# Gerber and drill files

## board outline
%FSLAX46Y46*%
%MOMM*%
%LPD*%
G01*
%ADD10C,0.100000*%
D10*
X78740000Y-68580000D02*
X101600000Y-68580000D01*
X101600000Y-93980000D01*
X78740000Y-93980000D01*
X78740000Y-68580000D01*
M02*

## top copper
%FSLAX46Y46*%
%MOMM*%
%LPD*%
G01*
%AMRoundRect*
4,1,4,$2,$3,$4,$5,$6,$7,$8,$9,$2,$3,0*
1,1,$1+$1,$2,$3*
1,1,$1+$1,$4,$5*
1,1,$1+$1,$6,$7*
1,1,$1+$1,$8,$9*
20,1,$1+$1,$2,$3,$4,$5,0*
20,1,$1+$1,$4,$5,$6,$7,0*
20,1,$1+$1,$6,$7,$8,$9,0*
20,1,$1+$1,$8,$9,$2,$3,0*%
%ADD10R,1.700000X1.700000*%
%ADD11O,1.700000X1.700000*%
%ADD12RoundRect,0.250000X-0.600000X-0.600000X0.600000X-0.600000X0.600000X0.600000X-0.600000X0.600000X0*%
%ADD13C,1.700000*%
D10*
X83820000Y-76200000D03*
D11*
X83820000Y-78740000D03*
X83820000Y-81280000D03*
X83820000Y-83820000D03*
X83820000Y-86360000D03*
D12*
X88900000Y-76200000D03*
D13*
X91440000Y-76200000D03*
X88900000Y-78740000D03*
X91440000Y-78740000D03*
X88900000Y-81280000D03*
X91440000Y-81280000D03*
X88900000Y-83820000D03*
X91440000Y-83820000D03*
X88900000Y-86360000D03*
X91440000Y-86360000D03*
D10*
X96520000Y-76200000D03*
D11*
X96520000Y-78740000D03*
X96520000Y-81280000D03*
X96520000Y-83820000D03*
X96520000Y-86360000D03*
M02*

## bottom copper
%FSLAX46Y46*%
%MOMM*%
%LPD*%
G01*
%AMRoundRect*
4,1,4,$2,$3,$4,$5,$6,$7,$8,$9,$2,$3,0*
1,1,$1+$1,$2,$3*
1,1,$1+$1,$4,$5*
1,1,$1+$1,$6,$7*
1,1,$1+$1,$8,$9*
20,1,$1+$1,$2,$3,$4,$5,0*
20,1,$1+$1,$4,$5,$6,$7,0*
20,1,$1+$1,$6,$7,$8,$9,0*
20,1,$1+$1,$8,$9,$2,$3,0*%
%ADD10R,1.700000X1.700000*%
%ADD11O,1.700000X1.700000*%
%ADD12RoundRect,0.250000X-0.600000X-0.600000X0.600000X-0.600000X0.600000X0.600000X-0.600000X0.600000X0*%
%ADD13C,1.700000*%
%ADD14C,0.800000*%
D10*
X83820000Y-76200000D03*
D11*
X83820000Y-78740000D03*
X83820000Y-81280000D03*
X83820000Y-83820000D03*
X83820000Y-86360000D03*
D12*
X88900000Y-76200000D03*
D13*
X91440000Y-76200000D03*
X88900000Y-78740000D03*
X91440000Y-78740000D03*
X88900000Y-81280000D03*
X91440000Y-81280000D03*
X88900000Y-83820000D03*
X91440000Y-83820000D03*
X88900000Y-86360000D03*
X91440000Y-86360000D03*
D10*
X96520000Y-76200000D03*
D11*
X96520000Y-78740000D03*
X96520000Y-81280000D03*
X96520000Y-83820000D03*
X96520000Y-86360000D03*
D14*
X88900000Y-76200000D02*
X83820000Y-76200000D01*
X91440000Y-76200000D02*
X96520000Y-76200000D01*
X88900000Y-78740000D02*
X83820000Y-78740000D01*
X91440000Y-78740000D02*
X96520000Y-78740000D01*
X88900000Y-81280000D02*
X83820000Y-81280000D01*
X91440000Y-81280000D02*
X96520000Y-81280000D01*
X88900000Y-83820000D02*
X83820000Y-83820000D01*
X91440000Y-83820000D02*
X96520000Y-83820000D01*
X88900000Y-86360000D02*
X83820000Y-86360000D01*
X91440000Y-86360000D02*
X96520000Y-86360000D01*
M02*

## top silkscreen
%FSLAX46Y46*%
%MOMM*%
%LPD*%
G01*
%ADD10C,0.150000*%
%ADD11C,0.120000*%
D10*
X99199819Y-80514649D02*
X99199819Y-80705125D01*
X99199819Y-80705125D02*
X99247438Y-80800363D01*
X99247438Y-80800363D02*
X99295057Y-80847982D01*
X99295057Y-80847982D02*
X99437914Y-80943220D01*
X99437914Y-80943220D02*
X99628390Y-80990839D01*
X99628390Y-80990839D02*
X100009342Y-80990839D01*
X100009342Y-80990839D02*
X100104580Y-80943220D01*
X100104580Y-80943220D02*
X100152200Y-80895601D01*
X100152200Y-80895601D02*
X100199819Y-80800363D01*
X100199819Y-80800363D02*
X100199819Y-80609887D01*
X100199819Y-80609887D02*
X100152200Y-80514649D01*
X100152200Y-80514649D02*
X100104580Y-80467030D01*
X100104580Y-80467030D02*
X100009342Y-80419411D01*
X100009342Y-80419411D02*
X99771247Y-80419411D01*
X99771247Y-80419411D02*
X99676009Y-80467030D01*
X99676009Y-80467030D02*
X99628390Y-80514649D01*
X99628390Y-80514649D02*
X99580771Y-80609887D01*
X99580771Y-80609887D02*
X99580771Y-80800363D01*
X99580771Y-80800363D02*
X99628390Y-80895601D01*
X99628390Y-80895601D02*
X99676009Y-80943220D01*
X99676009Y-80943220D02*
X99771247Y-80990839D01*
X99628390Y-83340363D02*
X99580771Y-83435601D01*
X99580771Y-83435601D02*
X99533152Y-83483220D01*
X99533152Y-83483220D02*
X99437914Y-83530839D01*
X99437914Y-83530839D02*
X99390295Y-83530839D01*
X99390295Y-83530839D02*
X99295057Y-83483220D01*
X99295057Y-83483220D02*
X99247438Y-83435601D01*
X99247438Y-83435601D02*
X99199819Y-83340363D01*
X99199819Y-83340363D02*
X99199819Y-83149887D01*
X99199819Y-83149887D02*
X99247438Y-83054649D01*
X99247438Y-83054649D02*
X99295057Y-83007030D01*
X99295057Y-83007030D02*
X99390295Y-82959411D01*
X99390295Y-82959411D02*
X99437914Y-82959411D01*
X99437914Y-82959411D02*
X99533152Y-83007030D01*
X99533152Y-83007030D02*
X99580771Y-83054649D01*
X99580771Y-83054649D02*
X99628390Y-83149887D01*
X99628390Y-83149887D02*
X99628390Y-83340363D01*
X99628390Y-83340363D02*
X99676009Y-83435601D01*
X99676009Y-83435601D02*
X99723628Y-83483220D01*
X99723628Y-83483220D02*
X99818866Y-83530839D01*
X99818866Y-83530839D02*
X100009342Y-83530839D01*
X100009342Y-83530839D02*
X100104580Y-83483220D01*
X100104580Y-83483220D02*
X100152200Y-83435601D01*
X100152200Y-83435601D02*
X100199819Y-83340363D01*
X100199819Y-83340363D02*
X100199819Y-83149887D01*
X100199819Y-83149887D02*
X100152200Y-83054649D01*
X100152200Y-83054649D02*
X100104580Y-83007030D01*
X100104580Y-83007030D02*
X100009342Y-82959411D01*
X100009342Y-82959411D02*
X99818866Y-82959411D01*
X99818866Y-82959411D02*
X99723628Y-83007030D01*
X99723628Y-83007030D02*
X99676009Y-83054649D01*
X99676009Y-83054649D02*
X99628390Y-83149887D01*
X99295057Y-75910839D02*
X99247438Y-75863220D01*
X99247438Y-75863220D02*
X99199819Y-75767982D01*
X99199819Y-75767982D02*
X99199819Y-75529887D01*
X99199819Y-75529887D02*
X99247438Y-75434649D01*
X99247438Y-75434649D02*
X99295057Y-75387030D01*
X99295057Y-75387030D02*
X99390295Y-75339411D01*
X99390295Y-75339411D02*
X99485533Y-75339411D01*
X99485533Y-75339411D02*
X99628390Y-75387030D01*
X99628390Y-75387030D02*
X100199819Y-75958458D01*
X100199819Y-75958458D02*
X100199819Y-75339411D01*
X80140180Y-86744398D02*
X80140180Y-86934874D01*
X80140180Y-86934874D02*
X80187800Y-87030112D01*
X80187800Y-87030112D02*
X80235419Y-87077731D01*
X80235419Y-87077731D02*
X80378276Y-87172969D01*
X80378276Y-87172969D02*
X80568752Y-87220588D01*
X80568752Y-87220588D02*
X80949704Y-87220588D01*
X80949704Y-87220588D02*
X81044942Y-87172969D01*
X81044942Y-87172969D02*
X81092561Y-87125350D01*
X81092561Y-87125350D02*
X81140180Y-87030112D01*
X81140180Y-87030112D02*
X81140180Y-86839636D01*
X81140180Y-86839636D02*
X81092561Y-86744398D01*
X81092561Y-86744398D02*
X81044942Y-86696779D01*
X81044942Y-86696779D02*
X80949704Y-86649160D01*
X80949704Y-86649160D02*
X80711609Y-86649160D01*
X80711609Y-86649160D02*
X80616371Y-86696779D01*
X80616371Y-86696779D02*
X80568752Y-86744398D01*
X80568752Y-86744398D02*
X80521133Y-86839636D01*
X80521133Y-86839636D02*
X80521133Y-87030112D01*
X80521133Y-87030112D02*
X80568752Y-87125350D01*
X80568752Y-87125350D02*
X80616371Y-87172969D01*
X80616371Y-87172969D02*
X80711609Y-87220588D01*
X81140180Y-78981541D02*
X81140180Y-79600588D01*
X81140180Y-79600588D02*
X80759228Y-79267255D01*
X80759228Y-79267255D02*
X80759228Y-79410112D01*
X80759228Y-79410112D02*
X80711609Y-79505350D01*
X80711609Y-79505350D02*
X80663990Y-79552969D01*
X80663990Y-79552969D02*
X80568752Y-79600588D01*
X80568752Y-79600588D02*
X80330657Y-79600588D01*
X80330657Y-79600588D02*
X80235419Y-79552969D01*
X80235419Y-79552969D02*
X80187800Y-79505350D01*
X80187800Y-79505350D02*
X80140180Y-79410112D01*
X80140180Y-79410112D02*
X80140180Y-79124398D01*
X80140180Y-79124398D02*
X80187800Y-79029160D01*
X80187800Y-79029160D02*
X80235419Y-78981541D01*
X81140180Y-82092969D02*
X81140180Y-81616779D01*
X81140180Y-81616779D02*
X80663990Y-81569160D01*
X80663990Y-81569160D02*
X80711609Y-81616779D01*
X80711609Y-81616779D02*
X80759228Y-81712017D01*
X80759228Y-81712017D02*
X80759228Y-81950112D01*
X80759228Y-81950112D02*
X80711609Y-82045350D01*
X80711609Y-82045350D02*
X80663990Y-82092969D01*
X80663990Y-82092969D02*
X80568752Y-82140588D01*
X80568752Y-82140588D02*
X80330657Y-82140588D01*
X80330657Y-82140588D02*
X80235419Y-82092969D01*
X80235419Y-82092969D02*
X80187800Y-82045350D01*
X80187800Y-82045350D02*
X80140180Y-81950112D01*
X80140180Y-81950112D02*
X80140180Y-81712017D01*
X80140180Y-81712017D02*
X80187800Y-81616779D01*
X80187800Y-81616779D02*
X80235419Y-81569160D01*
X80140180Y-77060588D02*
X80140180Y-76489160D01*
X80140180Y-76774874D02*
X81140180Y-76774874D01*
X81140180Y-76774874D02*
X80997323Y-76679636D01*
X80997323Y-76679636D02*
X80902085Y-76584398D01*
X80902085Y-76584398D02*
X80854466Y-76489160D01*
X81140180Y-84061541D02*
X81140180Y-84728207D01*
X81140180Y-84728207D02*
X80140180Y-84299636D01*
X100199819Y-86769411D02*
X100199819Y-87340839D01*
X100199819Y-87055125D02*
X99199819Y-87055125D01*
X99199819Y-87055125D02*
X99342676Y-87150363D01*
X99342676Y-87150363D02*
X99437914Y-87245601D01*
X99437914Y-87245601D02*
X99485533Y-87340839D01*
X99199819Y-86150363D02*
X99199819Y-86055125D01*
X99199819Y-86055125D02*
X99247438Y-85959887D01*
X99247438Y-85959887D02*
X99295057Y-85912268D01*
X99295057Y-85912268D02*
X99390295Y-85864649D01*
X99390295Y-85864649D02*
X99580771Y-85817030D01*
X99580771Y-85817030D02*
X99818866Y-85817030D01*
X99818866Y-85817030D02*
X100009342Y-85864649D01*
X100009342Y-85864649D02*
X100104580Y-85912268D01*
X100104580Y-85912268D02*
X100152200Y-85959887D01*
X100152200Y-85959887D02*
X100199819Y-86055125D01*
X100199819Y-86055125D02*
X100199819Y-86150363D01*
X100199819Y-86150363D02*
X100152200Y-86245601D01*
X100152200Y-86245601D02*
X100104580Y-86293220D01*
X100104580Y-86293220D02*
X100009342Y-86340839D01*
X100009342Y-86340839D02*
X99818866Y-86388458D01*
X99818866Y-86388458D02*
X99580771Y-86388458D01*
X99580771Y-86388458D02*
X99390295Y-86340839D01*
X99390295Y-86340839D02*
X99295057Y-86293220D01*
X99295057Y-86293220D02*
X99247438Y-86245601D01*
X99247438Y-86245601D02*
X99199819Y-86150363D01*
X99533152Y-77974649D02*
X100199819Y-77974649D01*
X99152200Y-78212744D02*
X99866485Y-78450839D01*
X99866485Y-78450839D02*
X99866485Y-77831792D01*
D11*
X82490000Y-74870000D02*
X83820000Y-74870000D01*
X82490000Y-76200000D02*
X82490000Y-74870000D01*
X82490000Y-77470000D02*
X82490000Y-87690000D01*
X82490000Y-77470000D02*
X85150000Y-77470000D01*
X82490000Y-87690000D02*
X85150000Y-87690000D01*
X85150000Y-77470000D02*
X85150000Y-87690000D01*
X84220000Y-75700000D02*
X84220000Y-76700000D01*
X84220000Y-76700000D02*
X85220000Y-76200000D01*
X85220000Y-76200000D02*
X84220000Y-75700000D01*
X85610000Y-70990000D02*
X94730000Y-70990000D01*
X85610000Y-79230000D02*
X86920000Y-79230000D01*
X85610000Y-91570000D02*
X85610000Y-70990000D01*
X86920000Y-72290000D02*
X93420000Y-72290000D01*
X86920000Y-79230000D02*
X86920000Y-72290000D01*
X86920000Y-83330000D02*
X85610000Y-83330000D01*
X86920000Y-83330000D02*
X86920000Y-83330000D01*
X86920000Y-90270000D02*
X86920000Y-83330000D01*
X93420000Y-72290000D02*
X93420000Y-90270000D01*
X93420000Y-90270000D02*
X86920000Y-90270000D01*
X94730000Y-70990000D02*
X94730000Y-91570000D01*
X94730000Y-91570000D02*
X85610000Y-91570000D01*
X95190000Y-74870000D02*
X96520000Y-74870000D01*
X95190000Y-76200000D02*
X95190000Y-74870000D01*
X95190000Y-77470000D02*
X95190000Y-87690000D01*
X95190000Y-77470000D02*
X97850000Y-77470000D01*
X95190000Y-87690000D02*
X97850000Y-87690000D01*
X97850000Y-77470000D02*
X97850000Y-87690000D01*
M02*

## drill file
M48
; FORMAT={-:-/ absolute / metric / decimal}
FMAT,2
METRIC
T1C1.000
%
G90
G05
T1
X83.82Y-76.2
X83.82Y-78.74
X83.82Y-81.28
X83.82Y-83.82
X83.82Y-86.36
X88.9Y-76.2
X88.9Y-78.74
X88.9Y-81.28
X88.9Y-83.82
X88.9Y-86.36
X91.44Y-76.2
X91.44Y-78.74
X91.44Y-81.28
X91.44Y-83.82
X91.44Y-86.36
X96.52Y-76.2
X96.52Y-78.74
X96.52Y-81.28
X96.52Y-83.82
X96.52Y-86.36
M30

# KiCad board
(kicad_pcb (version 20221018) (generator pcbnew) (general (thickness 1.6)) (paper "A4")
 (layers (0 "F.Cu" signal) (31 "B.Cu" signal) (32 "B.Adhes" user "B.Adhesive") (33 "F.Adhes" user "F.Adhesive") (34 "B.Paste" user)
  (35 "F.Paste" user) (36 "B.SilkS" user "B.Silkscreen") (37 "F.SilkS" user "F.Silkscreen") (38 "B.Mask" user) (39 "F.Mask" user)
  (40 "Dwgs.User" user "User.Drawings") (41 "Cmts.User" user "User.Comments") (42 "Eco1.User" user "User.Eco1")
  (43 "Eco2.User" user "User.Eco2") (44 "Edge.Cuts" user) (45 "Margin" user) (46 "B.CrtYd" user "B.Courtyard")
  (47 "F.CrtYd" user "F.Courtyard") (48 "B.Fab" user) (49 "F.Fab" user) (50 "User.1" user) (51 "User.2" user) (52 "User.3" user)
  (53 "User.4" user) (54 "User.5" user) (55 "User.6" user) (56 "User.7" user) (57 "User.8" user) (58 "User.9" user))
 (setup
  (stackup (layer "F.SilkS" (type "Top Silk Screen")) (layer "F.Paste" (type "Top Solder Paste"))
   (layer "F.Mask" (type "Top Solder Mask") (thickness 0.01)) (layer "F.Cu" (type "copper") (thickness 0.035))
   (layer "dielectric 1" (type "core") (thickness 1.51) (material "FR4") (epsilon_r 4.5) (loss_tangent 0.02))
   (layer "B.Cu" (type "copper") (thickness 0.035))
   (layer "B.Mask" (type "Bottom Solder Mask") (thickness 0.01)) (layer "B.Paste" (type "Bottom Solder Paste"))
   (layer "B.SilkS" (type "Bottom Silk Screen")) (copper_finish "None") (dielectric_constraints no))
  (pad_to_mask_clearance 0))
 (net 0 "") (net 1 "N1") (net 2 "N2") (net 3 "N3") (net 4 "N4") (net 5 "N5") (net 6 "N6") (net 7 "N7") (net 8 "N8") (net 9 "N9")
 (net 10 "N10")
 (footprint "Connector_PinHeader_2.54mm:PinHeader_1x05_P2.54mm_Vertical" (layer "F.Cu") (at 83.82 76.2)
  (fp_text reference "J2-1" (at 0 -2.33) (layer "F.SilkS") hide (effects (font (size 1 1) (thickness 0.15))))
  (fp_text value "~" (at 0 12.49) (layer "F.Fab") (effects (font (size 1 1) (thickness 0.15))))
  (fp_line (start -1.33 -1.33) (end 0 -1.33) (stroke (width 0.12) (type solid)) (layer "F.SilkS"))
  (fp_line (start -1.33 0) (end -1.33 -1.33) (stroke (width 0.12) (type solid)) (layer "F.SilkS"))
  (fp_line (start -1.33 1.27) (end -1.33 11.49) (stroke (width 0.12) (type solid)) (layer "F.SilkS"))
  (fp_line (start -1.33 1.27) (end 1.33 1.27) (stroke (width 0.12) (type solid)) (layer "F.SilkS"))
  (fp_line (start -1.33 11.49) (end 1.33 11.49) (stroke (width 0.12) (type solid)) (layer "F.SilkS"))
  (fp_line (start 1.33 1.27) (end 1.33 11.49) (stroke (width 0.12) (type solid)) (layer "F.SilkS"))
  (pad "1" thru_hole rect (at 0 0) (size 1.7 1.7) (drill 1) (layers "*.Cu" "*.Mask") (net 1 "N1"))
  (pad "2" thru_hole oval (at 0 2.54) (size 1.7 1.7) (drill 1) (layers "*.Cu" "*.Mask") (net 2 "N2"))
  (pad "3" thru_hole oval (at 0 5.08) (size 1.7 1.7) (drill 1) (layers "*.Cu" "*.Mask") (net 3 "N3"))
  (pad "4" thru_hole oval (at 0 7.62) (size 1.7 1.7) (drill 1) (layers "*.Cu" "*.Mask") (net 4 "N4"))
  (pad "5" thru_hole oval (at 0 10.16) (size 1.7 1.7) (drill 1) (layers "*.Cu" "*.Mask") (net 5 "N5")))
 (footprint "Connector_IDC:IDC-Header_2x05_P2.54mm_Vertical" (layer "F.Cu") (at 88.9 76.2)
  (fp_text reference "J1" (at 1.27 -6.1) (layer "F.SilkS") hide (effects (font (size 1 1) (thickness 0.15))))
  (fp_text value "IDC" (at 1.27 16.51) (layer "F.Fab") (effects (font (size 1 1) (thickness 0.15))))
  (fp_line (start -4.68 -0.5) (end -4.68 0.5) (stroke (width 0.12) (type solid)) (layer "F.SilkS"))
  (fp_line (start -4.68 0.5) (end -3.68 0) (stroke (width 0.12) (type solid)) (layer "F.SilkS"))
  (fp_line (start -3.68 0) (end -4.68 -0.5) (stroke (width 0.12) (type solid)) (layer "F.SilkS"))
  (fp_line (start -3.29 -5.21) (end 5.83 -5.21) (stroke (width 0.12) (type solid)) (layer "F.SilkS"))
  (fp_line (start -3.29 3.03) (end -1.98 3.03) (stroke (width 0.12) (type solid)) (layer "F.SilkS"))
  (fp_line (start -3.29 15.37) (end -3.29 -5.21) (stroke (width 0.12) (type solid)) (layer "F.SilkS"))
  (fp_line (start -1.98 -3.91) (end 4.52 -3.91) (stroke (width 0.12) (type solid)) (layer "F.SilkS"))
  (fp_line (start -1.98 3.03) (end -1.98 -3.91) (stroke (width 0.12) (type solid)) (layer "F.SilkS"))
  (fp_line (start -1.98 7.13) (end -3.29 7.13) (stroke (width 0.12) (type solid)) (layer "F.SilkS"))
  (fp_line (start -1.98 7.13) (end -1.98 7.13) (stroke (width 0.12) (type solid)) (layer "F.SilkS"))
  (fp_line (start -1.98 14.07) (end -1.98 7.13) (stroke (width 0.12) (type solid)) (layer "F.SilkS"))
  (fp_line (start 4.52 -3.91) (end 4.52 14.07) (stroke (width 0.12) (type solid)) (layer "F.SilkS"))
  (fp_line (start 4.52 14.07) (end -1.98 14.07) (stroke (width 0.12) (type solid)) (layer "F.SilkS"))
  (fp_line (start 5.83 -5.21) (end 5.83 15.37) (stroke (width 0.12) (type solid)) (layer "F.SilkS"))
  (fp_line (start 5.83 15.37) (end -3.29 15.37) (stroke (width 0.12) (type solid)) (layer "F.SilkS"))
  (pad "1" thru_hole roundrect (at 0 0) (size 1.7 1.7) (drill 1) (layers "*.Cu" "*.Mask") (roundrect_rratio 0.147059) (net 1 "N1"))
  (pad "2" thru_hole circle (at 2.54 0) (size 1.7 1.7) (drill 1) (layers "*.Cu" "*.Mask") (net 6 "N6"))
  (pad "3" thru_hole circle (at 0 2.54) (size 1.7 1.7) (drill 1) (layers "*.Cu" "*.Mask") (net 2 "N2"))
  (pad "4" thru_hole circle (at 2.54 2.54) (size 1.7 1.7) (drill 1) (layers "*.Cu" "*.Mask") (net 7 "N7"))
  (pad "5" thru_hole circle (at 0 5.08) (size 1.7 1.7) (drill 1) (layers "*.Cu" "*.Mask") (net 3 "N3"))
  (pad "6" thru_hole circle (at 2.54 5.08) (size 1.7 1.7) (drill 1) (layers "*.Cu" "*.Mask") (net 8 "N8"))
  (pad "7" thru_hole circle (at 0 7.62) (size 1.7 1.7) (drill 1) (layers "*.Cu" "*.Mask") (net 4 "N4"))
  (pad "8" thru_hole circle (at 2.54 7.62) (size 1.7 1.7) (drill 1) (layers "*.Cu" "*.Mask") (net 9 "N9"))
  (pad "9" thru_hole circle (at 0 10.16) (size 1.7 1.7) (drill 1) (layers "*.Cu" "*.Mask") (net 5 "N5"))
  (pad "10" thru_hole circle (at 2.54 10.16) (size 1.7 1.7) (drill 1) (layers "*.Cu" "*.Mask") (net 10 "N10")))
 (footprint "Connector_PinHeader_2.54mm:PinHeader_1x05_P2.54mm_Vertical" (layer "F.Cu") (at 96.52 76.2)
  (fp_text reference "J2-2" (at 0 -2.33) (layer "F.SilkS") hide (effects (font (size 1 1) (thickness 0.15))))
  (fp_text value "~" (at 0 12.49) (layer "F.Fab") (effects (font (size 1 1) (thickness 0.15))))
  (fp_line (start -1.33 -1.33) (end 0 -1.33) (stroke (width 0.12) (type solid)) (layer "F.SilkS"))
  (fp_line (start -1.33 0) (end -1.33 -1.33) (stroke (width 0.12) (type solid)) (layer "F.SilkS"))
  (fp_line (start -1.33 1.27) (end -1.33 11.49) (stroke (width 0.12) (type solid)) (layer "F.SilkS"))
  (fp_line (start -1.33 1.27) (end 1.33 1.27) (stroke (width 0.12) (type solid)) (layer "F.SilkS"))
  (fp_line (start -1.33 11.49) (end 1.33 11.49) (stroke (width 0.12) (type solid)) (layer "F.SilkS"))
  (fp_line (start 1.33 1.27) (end 1.33 11.49) (stroke (width 0.12) (type solid)) (layer "F.SilkS"))
  (pad "1" thru_hole rect (at 0 0) (size 1.7 1.7) (drill 1) (layers "*.Cu" "*.Mask") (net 6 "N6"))
  (pad "2" thru_hole oval (at 0 2.54) (size 1.7 1.7) (drill 1) (layers "*.Cu" "*.Mask") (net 7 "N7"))
  (pad "3" thru_hole oval (at 0 5.08) (size 1.7 1.7) (drill 1) (layers "*.Cu" "*.Mask") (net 8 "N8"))
  (pad "4" thru_hole oval (at 0 7.62) (size 1.7 1.7) (drill 1) (layers "*.Cu" "*.Mask") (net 9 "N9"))
  (pad "5" thru_hole oval (at 0 10.16) (size 1.7 1.7) (drill 1) (layers "*.Cu" "*.Mask") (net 10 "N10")))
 (gr_rect (start 78.74 68.58) (end 101.6 93.98) (stroke (width 0.1) (type default)) (fill none) (layer "Edge.Cuts"))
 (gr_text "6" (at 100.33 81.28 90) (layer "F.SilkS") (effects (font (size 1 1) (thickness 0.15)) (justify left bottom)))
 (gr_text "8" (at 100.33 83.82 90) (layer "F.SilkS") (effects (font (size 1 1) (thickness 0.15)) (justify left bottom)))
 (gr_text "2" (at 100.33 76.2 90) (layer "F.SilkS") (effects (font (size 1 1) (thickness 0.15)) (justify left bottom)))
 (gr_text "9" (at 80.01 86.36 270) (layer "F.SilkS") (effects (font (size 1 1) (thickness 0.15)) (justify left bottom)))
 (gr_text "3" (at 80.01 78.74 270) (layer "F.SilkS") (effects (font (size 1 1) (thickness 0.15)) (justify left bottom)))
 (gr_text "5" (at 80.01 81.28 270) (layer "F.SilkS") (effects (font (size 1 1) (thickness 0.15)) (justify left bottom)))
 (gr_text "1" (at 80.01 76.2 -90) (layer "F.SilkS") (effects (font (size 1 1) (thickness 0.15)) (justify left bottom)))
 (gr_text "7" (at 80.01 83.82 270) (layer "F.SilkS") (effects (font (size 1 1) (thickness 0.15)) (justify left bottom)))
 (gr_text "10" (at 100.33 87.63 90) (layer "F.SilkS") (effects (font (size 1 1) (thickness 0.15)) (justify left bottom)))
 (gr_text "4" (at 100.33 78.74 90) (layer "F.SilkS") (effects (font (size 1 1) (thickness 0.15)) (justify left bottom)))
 (segment (start 88.9 76.2) (end 83.82 76.2) (width 0.8) (layer "B.Cu") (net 1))
 (segment (start 91.44 76.2) (end 96.52 76.2) (width 0.8) (layer "B.Cu") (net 6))
 (segment (start 88.9 78.74) (end 83.82 78.74) (width 0.8) (layer "B.Cu") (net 2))
 (segment (start 91.44 78.74) (end 96.52 78.74) (width 0.8) (layer "B.Cu") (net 7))
 (segment (start 88.9 81.28) (end 83.82 81.28) (width 0.8) (layer "B.Cu") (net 3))
 (segment (start 91.44 81.28) (end 96.52 81.28) (width 0.8) (layer "B.Cu") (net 8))
 (segment (start 88.9 83.82) (end 83.82 83.82) (width 0.8) (layer "B.Cu") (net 4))
 (segment (start 91.44 83.82) (end 96.52 83.82) (width 0.8) (layer "B.Cu") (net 9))
 (segment (start 88.9 86.36) (end 83.82 86.36) (width 0.8) (layer "B.Cu") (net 5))
 (segment (start 91.44 86.36) (end 96.52 86.36) (width 0.8) (layer "B.Cu") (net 10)))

